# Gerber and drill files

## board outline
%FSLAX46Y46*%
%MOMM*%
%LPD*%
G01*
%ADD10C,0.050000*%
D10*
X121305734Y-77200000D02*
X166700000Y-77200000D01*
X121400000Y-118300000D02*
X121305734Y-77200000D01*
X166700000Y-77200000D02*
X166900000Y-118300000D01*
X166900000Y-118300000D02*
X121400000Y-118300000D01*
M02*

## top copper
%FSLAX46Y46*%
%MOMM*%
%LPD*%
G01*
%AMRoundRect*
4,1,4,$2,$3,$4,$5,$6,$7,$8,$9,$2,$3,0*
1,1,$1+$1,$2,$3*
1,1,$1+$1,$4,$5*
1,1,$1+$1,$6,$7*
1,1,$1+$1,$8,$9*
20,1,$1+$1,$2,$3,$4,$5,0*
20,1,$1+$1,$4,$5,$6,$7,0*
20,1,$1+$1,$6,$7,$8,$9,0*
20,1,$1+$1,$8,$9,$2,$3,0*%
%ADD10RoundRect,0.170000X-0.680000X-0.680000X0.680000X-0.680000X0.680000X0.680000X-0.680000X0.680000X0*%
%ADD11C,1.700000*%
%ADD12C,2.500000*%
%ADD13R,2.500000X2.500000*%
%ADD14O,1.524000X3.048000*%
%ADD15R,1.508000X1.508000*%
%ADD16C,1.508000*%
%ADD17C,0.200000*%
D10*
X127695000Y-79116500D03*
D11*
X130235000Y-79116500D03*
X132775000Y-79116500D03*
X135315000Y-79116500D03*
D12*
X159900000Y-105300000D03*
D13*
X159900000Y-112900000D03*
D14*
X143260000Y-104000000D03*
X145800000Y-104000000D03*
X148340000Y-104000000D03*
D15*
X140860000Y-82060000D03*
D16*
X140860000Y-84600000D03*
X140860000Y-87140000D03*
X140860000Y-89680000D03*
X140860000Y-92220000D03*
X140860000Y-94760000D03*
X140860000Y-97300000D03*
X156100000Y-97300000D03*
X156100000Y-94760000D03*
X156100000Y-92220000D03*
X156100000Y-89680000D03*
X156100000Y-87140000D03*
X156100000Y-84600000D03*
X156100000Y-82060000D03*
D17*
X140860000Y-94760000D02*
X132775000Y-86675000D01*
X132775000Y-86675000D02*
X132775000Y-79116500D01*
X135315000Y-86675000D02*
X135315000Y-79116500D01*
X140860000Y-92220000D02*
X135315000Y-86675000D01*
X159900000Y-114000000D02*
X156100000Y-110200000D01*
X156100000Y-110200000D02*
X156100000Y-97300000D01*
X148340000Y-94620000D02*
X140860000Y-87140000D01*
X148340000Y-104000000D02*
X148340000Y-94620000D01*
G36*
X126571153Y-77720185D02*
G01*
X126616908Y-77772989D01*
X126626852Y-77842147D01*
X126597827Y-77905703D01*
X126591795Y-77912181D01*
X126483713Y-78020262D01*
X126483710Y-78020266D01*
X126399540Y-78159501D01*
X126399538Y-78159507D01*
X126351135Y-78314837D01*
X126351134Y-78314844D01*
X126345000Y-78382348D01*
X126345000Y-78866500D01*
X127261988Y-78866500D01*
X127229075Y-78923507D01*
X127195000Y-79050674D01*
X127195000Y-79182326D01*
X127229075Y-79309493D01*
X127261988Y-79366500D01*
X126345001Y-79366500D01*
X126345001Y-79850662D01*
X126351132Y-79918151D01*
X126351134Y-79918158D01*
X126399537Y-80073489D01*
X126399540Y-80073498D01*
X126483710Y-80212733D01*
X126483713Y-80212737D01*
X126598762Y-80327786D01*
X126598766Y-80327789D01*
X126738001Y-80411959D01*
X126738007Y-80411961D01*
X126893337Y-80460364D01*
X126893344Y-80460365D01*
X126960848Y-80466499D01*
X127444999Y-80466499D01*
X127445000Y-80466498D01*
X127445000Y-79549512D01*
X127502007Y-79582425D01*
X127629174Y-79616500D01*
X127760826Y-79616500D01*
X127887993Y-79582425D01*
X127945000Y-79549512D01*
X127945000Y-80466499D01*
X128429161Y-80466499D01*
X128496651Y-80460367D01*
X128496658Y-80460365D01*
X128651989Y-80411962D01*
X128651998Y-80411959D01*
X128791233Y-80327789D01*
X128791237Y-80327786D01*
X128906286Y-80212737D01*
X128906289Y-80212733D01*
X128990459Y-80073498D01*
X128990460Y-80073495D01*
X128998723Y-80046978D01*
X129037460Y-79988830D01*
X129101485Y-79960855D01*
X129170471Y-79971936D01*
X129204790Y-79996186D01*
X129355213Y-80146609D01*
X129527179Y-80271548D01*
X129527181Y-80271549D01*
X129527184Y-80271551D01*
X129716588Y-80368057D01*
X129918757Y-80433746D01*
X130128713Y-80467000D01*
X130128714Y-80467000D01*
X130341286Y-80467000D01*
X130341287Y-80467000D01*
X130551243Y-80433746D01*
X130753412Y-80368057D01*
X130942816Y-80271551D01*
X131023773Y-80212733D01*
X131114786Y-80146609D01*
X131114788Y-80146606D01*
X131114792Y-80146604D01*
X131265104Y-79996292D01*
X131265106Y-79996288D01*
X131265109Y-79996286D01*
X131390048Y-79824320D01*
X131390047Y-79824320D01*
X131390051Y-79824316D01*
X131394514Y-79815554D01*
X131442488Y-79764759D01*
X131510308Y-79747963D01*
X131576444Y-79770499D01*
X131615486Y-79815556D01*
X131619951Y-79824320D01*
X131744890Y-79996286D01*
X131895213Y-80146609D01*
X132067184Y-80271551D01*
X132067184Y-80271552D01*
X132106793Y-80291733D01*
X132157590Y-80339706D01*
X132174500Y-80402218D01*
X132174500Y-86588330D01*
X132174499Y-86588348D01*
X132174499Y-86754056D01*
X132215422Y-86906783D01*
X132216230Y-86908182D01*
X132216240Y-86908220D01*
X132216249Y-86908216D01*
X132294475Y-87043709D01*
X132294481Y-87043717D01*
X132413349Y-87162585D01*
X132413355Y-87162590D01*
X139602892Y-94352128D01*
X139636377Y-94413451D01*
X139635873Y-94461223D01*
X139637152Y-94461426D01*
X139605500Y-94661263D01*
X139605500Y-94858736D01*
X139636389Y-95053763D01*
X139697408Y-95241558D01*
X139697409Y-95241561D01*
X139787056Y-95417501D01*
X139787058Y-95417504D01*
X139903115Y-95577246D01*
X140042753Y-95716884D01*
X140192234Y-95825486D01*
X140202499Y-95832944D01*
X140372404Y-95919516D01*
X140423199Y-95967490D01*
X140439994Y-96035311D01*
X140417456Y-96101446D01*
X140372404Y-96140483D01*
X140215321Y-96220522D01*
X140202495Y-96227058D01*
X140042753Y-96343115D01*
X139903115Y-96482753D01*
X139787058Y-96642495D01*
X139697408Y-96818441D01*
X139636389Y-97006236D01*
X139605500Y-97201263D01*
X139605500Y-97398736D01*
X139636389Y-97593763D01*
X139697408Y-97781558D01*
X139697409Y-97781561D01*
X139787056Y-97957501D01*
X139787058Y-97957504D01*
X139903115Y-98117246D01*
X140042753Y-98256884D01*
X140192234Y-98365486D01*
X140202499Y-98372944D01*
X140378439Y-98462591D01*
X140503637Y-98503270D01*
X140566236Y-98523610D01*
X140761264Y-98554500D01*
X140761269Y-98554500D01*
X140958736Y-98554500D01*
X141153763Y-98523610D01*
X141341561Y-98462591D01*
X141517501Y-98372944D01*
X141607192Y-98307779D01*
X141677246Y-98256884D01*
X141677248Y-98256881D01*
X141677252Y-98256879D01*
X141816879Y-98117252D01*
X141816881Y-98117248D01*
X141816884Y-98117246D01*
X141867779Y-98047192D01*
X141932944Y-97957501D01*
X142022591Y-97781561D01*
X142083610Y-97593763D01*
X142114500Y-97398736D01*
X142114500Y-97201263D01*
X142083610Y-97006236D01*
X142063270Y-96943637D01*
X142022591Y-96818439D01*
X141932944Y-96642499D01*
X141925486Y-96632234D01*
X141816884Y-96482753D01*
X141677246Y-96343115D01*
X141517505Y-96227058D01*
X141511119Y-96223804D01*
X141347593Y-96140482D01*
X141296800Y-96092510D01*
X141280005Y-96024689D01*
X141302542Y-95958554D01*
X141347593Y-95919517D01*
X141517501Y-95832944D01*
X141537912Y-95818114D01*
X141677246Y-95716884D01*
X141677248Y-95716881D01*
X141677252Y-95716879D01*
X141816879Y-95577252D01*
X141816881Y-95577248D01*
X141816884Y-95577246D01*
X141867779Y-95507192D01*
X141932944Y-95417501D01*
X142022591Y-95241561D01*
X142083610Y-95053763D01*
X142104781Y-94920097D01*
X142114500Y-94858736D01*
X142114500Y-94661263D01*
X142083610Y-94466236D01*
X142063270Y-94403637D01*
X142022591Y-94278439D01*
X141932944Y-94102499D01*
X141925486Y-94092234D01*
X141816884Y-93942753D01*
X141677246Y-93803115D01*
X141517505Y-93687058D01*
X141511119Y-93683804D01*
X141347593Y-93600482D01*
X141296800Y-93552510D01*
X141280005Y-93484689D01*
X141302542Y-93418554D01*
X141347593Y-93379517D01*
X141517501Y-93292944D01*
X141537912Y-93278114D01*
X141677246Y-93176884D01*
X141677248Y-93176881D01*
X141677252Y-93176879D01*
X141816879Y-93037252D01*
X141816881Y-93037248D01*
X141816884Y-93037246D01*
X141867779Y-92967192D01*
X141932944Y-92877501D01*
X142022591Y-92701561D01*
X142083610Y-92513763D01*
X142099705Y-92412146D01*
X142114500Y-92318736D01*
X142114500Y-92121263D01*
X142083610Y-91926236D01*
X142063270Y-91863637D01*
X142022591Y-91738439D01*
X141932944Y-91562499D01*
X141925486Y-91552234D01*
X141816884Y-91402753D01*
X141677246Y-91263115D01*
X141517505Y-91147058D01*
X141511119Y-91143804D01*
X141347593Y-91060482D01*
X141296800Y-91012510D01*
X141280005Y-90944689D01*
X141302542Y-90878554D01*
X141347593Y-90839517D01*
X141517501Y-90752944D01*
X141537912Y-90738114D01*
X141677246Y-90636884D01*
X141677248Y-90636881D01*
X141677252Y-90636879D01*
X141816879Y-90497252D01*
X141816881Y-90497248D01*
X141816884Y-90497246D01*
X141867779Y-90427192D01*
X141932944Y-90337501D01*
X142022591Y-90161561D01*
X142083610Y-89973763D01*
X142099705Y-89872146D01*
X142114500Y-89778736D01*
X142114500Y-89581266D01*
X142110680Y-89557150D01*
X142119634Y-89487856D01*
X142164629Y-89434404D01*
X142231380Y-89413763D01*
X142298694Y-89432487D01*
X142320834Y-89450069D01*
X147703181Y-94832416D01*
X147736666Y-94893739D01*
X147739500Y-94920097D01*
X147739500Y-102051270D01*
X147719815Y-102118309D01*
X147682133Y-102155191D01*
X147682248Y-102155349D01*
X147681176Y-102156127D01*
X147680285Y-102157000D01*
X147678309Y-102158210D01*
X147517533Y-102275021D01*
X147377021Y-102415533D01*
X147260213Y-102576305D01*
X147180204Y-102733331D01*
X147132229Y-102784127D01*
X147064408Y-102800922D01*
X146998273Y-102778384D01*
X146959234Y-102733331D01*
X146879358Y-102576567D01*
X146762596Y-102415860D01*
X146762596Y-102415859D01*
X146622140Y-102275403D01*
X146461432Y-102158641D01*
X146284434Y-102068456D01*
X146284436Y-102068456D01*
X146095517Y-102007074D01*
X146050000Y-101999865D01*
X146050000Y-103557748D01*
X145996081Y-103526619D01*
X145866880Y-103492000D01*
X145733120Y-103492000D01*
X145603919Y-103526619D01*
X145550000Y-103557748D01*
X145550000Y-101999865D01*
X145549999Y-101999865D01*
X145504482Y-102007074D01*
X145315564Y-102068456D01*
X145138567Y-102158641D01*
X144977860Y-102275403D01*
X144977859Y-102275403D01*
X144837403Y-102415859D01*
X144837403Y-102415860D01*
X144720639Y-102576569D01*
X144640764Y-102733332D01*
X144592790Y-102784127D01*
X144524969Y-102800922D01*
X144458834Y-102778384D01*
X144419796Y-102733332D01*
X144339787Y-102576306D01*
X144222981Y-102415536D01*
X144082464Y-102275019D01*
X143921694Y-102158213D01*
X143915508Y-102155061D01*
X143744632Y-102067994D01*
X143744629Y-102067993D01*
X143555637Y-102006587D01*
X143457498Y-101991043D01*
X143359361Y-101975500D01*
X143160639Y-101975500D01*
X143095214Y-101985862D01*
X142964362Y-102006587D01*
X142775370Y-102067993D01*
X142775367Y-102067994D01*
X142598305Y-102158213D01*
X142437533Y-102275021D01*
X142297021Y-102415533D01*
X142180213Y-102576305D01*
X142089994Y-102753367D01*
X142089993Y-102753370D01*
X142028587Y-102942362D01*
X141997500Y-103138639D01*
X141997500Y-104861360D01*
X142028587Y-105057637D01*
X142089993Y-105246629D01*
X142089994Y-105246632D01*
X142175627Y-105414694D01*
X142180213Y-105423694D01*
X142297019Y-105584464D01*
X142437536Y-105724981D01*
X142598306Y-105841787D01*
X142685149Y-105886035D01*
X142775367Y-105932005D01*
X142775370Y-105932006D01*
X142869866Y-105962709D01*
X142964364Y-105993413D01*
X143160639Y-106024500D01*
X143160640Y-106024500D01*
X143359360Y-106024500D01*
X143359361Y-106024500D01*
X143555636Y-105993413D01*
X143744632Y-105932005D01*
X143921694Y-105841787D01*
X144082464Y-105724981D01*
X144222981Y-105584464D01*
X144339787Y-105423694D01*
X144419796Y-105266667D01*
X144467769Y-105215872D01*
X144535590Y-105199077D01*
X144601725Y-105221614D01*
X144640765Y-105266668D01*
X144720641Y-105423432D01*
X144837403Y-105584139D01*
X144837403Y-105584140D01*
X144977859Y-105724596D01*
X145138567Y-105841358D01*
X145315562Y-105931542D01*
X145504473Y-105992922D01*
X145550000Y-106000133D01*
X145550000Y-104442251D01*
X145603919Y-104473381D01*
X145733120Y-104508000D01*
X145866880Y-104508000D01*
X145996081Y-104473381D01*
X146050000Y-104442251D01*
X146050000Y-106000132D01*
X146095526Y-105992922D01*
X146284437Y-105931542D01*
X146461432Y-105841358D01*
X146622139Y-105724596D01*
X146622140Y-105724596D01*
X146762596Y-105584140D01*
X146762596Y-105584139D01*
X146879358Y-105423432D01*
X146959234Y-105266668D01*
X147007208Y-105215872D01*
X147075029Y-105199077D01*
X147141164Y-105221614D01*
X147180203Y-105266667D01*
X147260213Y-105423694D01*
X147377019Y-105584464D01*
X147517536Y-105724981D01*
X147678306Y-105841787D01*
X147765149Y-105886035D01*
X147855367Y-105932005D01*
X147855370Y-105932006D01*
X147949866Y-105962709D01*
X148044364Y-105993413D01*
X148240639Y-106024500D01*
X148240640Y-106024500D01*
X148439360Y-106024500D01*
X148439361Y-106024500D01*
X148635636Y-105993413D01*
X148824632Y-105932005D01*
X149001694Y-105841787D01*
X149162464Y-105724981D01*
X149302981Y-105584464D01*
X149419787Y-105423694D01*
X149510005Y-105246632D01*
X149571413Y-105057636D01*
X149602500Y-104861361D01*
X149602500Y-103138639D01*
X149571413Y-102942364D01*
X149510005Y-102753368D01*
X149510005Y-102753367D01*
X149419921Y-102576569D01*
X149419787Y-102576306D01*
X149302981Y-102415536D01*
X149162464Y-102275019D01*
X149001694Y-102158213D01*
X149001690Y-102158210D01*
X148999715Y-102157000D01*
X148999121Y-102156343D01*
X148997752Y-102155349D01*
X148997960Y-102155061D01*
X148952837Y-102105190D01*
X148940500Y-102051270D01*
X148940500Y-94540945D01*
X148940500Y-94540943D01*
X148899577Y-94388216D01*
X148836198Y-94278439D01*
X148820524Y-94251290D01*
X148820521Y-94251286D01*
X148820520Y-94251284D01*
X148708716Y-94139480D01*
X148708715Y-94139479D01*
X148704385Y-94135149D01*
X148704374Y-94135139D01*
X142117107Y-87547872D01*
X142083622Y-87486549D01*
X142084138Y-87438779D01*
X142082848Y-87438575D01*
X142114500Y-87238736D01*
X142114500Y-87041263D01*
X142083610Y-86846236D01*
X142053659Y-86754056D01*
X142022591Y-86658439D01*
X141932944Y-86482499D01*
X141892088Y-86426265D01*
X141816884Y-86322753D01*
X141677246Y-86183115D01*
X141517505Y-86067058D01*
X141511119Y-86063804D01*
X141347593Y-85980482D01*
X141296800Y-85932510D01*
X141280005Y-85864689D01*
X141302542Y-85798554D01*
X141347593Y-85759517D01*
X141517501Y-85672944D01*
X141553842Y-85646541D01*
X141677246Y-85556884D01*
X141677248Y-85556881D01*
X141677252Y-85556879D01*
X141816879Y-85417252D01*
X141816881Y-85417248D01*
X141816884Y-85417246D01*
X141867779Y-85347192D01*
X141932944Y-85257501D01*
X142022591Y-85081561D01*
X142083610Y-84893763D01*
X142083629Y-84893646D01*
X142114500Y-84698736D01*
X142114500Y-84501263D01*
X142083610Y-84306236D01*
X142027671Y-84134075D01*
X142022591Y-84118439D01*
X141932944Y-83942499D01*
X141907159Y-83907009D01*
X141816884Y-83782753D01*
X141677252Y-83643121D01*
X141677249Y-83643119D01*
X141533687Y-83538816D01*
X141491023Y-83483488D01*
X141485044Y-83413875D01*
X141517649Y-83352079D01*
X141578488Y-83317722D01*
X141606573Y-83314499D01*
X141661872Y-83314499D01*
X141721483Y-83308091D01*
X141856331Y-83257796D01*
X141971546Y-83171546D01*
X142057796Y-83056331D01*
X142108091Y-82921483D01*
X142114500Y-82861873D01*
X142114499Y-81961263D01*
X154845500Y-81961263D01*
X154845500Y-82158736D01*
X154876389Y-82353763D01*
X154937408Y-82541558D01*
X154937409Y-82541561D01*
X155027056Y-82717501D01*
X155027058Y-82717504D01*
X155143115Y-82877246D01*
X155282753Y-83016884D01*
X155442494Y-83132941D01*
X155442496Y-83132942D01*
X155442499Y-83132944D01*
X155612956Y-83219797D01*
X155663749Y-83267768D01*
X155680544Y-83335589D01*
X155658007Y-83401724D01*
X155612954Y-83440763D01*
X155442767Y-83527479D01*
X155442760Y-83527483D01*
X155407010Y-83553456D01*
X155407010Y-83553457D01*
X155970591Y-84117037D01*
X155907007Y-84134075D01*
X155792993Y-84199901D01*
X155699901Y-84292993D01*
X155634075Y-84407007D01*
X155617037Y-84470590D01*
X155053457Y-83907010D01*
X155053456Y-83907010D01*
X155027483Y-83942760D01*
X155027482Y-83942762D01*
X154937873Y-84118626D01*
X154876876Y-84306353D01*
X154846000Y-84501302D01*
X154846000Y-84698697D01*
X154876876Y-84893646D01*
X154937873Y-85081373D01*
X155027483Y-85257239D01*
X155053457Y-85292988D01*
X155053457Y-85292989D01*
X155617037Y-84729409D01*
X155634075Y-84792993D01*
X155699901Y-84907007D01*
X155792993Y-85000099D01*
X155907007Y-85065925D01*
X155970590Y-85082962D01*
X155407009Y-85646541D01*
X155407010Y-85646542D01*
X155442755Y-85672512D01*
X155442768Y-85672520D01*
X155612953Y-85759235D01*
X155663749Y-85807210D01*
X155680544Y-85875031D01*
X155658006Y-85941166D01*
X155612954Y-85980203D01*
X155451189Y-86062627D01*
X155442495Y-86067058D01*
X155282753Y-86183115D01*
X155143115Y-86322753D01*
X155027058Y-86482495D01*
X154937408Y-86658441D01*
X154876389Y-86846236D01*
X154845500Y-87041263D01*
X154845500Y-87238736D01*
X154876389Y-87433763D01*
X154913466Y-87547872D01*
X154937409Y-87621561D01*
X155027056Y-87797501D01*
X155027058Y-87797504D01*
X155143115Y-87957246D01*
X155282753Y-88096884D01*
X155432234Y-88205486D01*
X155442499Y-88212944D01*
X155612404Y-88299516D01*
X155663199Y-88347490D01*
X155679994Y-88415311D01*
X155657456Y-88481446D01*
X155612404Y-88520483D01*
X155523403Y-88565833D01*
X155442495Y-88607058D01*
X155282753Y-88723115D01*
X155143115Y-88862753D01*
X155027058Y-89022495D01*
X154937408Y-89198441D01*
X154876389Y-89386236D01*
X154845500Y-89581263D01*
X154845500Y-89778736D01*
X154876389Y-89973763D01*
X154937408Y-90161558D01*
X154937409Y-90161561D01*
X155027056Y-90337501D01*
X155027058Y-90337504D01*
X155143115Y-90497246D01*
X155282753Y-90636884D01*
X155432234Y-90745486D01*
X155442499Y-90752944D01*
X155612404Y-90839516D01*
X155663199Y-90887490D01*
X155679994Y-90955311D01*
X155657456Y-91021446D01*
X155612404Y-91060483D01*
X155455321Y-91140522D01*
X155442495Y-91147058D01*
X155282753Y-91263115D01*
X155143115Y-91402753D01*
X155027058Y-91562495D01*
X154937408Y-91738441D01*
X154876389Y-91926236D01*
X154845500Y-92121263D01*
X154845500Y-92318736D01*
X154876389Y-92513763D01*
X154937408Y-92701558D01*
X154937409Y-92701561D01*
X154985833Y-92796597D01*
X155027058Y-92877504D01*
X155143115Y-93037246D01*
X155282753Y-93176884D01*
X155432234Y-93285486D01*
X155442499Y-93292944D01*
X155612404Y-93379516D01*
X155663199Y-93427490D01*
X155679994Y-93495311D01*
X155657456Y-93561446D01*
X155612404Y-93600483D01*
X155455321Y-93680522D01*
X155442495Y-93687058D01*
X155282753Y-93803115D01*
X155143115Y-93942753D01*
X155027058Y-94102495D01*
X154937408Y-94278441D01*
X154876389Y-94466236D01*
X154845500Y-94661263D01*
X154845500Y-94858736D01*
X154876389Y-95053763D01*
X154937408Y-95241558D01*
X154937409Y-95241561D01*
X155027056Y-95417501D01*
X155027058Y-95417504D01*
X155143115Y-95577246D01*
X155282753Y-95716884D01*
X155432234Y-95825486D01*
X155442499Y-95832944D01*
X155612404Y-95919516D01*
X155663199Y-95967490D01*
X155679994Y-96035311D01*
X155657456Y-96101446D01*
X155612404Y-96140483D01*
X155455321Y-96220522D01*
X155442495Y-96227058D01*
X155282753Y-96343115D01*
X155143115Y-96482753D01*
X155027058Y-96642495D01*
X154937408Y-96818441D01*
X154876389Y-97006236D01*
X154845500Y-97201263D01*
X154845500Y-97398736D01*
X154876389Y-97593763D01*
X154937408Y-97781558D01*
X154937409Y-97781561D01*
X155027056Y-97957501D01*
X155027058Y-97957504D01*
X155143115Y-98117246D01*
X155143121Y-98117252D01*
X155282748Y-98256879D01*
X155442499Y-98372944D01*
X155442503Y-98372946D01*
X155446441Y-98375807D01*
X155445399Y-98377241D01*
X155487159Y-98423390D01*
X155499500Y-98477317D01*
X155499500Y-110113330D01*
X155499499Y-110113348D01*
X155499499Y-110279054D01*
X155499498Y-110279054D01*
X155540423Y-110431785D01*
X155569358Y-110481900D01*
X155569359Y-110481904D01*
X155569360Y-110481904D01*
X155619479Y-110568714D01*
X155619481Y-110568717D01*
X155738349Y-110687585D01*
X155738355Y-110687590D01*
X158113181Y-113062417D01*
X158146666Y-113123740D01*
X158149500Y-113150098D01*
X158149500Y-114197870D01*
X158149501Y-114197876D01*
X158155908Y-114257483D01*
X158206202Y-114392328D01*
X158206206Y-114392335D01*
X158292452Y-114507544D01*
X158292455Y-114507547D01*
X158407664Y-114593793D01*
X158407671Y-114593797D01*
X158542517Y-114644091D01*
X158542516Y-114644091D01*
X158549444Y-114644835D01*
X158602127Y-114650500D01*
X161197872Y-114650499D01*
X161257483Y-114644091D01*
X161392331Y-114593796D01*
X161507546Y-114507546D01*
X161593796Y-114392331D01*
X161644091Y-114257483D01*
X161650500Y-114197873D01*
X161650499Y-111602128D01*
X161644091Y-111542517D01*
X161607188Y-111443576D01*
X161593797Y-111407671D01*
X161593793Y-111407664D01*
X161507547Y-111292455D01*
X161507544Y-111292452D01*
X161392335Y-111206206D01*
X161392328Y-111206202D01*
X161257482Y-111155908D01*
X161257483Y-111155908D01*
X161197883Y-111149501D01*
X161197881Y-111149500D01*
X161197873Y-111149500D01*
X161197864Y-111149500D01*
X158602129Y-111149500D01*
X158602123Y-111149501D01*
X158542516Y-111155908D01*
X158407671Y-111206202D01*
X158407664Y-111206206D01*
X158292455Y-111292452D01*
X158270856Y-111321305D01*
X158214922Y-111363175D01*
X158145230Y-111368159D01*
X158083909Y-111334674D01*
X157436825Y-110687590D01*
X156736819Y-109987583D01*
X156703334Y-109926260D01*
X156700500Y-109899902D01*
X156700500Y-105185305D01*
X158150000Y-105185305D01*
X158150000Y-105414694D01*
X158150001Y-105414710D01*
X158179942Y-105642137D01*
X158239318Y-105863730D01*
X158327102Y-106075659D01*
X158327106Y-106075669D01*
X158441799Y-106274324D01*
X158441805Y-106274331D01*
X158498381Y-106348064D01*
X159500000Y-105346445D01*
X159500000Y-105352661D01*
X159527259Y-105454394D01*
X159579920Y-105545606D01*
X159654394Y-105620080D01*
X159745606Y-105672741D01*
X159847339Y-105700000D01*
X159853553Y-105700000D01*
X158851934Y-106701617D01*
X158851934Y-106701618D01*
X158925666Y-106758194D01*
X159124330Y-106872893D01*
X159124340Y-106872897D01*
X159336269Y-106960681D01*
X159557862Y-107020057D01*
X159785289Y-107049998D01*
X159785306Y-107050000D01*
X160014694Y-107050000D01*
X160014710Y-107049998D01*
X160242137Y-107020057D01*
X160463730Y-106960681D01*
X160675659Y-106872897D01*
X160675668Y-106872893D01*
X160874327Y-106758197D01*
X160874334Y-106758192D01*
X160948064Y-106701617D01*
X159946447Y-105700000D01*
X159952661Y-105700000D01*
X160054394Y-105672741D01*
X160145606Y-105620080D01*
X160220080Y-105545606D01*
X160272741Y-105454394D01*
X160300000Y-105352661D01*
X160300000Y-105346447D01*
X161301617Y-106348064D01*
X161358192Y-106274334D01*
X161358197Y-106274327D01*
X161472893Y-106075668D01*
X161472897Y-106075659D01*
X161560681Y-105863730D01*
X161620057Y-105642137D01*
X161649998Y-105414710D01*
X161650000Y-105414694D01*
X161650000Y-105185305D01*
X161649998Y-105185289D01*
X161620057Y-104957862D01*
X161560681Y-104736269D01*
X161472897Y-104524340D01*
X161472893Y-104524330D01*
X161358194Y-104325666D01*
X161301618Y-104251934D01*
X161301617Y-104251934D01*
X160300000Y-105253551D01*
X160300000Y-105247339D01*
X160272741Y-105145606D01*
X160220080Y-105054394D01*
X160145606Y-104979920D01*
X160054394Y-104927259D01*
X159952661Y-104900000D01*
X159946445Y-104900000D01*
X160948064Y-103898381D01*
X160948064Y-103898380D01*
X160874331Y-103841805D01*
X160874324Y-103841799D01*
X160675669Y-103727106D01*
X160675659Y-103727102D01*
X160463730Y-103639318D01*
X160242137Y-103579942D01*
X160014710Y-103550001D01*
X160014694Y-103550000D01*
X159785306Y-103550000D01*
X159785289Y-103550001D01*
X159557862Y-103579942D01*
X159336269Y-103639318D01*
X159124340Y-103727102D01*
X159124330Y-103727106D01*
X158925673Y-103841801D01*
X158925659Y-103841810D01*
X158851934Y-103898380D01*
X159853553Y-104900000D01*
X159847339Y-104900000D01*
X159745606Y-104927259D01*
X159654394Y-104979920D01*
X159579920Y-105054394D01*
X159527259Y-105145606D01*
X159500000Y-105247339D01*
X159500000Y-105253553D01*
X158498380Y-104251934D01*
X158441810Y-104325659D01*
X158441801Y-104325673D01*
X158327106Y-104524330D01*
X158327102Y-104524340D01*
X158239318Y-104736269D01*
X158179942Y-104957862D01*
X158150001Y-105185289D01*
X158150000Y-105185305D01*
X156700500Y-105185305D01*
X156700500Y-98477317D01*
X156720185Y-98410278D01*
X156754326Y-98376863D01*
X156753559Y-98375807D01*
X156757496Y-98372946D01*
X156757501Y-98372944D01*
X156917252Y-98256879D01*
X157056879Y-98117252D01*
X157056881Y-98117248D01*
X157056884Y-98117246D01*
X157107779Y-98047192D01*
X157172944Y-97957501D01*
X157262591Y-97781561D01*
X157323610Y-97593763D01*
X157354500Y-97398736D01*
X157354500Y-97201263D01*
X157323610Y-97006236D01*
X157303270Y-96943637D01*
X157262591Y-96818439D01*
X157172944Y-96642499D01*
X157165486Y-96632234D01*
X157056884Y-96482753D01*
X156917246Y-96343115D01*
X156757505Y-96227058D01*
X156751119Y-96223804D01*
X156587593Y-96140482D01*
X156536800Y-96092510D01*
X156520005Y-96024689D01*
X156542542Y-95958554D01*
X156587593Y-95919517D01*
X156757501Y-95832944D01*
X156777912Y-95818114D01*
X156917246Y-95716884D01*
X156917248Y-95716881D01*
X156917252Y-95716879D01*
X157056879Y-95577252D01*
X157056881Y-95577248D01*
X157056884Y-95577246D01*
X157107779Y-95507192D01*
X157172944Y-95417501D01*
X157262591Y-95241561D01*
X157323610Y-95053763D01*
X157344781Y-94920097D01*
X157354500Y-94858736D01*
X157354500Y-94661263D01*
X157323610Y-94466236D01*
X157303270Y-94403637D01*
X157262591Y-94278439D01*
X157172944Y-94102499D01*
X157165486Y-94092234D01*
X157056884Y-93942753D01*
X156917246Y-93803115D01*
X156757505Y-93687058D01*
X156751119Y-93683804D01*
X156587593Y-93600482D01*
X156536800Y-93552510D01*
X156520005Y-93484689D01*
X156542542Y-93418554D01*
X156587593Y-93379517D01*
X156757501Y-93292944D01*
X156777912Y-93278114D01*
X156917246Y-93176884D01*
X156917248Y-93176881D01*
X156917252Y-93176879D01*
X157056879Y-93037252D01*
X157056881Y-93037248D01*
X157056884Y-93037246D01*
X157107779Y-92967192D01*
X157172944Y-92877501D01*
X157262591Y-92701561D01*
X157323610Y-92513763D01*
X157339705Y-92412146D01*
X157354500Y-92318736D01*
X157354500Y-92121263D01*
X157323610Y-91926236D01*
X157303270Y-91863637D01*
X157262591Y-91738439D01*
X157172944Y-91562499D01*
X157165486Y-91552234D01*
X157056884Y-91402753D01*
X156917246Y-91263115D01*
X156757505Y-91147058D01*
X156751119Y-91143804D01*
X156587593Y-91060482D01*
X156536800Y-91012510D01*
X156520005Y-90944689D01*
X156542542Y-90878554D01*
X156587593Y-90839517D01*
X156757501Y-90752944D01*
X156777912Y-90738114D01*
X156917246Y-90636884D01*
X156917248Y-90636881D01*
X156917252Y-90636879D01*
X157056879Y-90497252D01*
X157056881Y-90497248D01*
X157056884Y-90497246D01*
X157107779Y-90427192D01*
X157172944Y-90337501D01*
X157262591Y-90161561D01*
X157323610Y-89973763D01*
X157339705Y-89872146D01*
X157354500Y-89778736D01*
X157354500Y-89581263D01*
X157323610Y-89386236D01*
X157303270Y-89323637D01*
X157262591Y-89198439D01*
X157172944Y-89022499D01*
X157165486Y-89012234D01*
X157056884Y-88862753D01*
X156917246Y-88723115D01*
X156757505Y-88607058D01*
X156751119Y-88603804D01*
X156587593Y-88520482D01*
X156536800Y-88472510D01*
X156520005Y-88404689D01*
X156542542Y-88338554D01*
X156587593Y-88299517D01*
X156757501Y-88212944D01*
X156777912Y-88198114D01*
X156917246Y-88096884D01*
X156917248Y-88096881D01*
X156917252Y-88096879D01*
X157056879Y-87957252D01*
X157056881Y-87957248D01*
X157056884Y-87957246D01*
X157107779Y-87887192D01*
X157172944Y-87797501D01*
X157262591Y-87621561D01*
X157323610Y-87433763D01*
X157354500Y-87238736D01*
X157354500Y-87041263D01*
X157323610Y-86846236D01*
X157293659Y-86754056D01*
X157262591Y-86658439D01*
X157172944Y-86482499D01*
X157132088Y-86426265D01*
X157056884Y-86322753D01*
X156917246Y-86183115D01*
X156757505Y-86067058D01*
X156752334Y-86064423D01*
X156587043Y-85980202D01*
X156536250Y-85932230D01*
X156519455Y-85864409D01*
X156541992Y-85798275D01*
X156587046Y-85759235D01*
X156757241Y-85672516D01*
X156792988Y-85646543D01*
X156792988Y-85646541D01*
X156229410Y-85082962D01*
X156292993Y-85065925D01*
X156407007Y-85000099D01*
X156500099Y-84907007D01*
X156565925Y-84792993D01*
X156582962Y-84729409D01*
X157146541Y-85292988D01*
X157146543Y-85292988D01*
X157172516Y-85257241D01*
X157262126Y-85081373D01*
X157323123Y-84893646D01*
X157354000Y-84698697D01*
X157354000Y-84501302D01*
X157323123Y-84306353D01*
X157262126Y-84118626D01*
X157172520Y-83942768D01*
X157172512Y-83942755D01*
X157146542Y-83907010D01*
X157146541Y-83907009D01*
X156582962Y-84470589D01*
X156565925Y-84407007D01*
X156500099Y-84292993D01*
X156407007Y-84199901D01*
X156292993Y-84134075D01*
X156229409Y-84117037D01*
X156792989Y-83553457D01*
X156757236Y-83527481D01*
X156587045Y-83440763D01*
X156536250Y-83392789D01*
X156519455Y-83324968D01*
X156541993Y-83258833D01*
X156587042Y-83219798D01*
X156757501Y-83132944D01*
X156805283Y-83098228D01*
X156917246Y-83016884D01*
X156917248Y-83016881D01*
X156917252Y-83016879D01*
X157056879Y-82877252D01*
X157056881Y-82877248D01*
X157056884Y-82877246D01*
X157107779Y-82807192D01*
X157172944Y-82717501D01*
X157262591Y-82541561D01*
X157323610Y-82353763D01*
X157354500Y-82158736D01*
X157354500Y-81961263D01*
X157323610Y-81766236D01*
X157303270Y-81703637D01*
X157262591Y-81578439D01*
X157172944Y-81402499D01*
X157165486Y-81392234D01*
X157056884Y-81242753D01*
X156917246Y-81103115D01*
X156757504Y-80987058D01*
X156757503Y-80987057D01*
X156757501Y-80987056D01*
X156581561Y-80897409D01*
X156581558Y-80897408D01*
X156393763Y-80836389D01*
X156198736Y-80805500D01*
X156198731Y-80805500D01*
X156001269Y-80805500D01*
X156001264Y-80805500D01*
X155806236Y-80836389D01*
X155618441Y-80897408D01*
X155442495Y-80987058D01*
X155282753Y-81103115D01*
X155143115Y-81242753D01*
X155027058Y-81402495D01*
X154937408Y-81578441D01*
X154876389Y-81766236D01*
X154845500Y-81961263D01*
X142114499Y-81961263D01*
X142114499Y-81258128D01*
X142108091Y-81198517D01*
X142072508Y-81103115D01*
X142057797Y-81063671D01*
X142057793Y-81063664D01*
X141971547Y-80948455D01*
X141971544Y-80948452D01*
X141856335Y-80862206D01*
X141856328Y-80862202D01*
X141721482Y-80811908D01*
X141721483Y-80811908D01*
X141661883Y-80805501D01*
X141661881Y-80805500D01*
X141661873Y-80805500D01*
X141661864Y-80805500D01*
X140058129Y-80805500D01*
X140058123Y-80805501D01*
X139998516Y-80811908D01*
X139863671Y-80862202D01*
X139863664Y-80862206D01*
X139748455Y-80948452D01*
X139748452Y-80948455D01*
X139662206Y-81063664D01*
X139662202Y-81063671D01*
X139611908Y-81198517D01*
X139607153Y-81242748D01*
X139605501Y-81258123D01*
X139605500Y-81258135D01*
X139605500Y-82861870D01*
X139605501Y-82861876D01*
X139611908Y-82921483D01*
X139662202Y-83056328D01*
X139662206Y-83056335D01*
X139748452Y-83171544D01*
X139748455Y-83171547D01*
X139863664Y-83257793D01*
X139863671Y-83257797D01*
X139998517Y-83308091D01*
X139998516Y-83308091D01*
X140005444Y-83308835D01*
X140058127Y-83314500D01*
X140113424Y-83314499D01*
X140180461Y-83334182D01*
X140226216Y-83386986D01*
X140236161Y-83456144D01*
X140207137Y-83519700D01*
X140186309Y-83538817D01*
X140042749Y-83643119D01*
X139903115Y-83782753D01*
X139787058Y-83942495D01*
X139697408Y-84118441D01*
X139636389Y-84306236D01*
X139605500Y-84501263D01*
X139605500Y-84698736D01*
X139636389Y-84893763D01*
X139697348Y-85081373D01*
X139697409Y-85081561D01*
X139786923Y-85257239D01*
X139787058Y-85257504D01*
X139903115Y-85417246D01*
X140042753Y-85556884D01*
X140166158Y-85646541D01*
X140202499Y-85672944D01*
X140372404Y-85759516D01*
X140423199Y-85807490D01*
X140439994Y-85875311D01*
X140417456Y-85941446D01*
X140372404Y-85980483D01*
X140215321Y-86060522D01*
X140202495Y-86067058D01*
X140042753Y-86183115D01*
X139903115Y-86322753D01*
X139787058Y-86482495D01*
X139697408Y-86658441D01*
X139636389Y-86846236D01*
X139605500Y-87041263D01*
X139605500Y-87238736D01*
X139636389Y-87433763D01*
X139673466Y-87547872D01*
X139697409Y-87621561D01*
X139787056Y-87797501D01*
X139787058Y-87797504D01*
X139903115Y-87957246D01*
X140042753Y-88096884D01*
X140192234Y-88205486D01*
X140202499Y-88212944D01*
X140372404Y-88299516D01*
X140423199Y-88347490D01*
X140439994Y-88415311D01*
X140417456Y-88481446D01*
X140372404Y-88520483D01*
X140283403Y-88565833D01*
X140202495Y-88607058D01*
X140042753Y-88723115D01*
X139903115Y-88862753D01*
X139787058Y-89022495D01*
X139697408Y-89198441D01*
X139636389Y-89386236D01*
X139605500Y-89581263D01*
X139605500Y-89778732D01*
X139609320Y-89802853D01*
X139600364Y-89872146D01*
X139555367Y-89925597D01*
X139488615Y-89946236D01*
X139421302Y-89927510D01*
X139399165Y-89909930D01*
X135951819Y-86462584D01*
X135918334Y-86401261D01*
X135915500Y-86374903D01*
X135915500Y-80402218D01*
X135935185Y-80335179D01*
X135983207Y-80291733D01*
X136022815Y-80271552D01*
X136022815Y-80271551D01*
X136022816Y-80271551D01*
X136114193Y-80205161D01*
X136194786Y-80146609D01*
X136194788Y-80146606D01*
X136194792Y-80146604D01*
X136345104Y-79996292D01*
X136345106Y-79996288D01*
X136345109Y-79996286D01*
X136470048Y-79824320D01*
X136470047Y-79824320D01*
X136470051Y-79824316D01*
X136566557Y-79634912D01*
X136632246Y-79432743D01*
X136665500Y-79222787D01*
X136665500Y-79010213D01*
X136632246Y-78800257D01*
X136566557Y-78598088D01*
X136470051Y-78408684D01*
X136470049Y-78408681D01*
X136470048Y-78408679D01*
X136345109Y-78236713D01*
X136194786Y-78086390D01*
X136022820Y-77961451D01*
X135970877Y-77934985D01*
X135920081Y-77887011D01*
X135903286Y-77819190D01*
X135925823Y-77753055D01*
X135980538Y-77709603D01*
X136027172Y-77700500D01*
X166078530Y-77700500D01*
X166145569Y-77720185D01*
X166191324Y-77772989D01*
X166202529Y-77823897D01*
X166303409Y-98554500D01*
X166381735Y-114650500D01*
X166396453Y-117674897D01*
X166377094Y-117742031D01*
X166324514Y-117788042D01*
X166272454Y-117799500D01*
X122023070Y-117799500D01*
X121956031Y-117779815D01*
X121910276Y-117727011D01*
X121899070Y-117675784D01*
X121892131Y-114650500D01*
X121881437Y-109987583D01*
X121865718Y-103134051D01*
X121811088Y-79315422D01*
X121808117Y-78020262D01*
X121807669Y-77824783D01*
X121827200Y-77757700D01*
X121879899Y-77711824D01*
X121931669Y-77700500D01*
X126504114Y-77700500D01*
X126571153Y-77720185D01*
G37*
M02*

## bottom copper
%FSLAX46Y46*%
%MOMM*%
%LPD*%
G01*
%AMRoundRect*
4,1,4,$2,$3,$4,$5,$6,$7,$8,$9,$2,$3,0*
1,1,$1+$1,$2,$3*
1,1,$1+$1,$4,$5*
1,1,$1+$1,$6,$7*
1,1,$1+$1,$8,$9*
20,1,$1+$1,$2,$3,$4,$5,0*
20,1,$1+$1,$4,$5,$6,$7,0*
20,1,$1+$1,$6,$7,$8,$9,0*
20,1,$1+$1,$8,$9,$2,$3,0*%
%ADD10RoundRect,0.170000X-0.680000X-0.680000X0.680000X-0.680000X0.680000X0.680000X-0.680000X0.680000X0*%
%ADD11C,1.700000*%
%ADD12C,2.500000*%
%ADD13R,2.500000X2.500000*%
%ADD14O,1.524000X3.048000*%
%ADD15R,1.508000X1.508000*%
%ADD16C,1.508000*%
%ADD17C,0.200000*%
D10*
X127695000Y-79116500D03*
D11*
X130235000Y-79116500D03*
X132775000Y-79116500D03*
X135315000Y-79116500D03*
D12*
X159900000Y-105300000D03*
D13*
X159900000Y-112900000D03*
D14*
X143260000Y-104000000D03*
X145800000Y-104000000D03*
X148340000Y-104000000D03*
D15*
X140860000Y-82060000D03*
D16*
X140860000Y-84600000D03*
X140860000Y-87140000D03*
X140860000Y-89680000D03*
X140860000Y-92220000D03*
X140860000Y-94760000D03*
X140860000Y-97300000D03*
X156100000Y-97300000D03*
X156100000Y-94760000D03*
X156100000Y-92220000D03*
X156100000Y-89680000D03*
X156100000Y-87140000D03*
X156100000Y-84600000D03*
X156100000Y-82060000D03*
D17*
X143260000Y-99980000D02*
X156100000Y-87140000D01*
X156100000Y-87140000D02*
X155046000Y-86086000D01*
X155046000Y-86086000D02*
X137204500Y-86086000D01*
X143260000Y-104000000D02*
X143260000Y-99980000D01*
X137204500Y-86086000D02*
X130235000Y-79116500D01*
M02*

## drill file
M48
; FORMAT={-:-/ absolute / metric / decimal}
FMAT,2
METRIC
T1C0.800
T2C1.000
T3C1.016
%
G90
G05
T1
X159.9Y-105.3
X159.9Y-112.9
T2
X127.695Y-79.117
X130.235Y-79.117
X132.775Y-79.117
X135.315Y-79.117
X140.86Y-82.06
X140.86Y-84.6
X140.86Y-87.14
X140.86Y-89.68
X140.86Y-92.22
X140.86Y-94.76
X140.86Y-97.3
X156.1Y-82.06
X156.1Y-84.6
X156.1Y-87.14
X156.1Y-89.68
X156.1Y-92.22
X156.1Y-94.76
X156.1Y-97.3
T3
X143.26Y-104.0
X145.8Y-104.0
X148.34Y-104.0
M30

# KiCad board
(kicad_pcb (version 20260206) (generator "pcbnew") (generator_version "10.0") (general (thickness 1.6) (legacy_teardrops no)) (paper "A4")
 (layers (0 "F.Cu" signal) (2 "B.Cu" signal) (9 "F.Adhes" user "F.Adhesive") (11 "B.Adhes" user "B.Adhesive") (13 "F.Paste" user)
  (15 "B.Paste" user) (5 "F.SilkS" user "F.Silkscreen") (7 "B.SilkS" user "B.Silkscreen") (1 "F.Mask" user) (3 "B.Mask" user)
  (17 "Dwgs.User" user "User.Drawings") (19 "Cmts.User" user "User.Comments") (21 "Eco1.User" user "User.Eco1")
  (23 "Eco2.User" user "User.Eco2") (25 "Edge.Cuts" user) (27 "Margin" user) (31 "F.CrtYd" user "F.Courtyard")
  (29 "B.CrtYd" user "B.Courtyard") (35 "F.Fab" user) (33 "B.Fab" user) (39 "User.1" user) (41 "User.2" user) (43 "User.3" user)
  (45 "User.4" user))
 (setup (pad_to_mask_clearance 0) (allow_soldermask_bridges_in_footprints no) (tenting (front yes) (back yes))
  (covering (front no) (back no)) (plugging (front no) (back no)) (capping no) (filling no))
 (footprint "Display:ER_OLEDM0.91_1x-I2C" (layer "F.Cu") (at 127.695 79.1165)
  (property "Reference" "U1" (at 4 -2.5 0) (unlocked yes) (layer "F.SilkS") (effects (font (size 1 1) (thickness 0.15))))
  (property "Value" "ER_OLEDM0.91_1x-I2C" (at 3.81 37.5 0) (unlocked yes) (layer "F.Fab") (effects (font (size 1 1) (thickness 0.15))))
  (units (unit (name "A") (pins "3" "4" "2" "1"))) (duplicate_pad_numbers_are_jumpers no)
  (pad "1" thru_hole roundrect (at 0 0) (size 1.7 1.7) (drill 1) (layers "*.Cu" "*.Mask") (remove_unused_layers no) (roundrect_rratio 0.1)
   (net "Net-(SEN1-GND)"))
  (pad "2" thru_hole circle (at 2.54 0) (size 1.7 1.7) (drill 1) (layers "*.Cu" "*.Mask") (remove_unused_layers no) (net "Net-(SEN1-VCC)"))
  (pad "3" thru_hole circle (at 5.08 0) (size 1.7 1.7) (drill 1) (layers "*.Cu" "*.Mask") (remove_unused_layers no) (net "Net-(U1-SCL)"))
  (pad "4" thru_hole circle (at 7.62 0) (size 1.7 1.7) (drill 1) (layers "*.Cu" "*.Mask") (remove_unused_layers no) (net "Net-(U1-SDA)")))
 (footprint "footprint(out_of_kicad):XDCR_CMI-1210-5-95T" (layer "F.Cu") (at 159.9 109.1 90)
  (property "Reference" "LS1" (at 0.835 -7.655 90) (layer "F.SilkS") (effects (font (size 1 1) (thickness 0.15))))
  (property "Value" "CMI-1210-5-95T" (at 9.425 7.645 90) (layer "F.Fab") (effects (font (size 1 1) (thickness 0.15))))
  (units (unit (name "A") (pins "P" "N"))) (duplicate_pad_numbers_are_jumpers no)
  (pad "N" thru_hole circle (at 3.8 0 90) (size 2.5 2.5) (drill 0.8) (layers "*.Cu" "*.Mask") (remove_unused_layers no)
   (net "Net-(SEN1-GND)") (solder_mask_margin 0.102))
  (pad "P" thru_hole rect (at -3.8 0 90) (size 2.5 2.5) (drill 0.8) (layers "*.Cu" "*.Mask") (remove_unused_layers no)
   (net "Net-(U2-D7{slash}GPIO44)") (solder_mask_margin 0.102)))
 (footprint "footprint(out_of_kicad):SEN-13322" (layer "F.Cu") (at 145.8 104)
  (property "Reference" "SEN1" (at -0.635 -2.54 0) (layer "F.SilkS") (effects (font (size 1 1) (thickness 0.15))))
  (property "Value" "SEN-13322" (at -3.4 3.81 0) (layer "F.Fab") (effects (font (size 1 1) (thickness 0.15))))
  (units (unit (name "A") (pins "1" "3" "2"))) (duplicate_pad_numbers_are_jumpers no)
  (pad "1" thru_hole oval (at -2.54 0) (size 1.524 3.048) (drill 1.016) (layers "*.Cu" "*.Mask") (remove_unused_layers no)
   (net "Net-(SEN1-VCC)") (solder_mask_margin 0.102))
  (pad "2" thru_hole oval (at 0 0) (size 1.524 3.048) (drill 1.016) (layers "*.Cu" "*.Mask") (remove_unused_layers no)
   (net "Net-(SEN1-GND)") (solder_mask_margin 0.102))
  (pad "3" thru_hole oval (at 2.54 0) (size 1.524 3.048) (drill 1.016) (layers "*.Cu" "*.Mask") (remove_unused_layers no)
   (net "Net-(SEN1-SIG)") (solder_mask_margin 0.102)))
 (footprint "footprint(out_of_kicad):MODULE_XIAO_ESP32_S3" (layer "F.Cu") (at 148.48 89.6165)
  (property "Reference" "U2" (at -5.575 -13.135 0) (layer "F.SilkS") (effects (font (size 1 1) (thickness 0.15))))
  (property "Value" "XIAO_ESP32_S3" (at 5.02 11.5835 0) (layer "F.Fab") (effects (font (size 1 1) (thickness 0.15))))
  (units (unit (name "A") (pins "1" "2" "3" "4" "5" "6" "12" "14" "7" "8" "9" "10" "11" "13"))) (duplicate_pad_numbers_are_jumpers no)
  (pad "1" thru_hole rect (at -7.62 -7.5565) (size 1.508 1.508) (drill 1) (layers "*.Cu" "*.Mask") (remove_unused_layers no)
   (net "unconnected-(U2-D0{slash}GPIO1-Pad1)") (solder_mask_margin 0.102))
  (pad "2" thru_hole circle (at -7.62 -5.0165) (size 1.508 1.508) (drill 1) (layers "*.Cu" "*.Mask") (remove_unused_layers no)
   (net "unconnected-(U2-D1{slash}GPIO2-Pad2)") (solder_mask_margin 0.102))
  (pad "3" thru_hole circle (at -7.62 -2.4765) (size 1.508 1.508) (drill 1) (layers "*.Cu" "*.Mask") (remove_unused_layers no)
   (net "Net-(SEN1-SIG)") (solder_mask_margin 0.102))
  (pad "4" thru_hole circle (at -7.62 0.0635) (size 1.508 1.508) (drill 1) (layers "*.Cu" "*.Mask") (remove_unused_layers no)
   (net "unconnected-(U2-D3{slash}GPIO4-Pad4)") (solder_mask_margin 0.102))
  (pad "5" thru_hole circle (at -7.62 2.6035) (size 1.508 1.508) (drill 1) (layers "*.Cu" "*.Mask") (remove_unused_layers no)
   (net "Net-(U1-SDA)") (solder_mask_margin 0.102))
  (pad "6" thru_hole circle (at -7.62 5.1435) (size 1.508 1.508) (drill 1) (layers "*.Cu" "*.Mask") (remove_unused_layers no)
   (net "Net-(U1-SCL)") (solder_mask_margin 0.102))
  (pad "7" thru_hole circle (at -7.62 7.6835) (size 1.508 1.508) (drill 1) (layers "*.Cu" "*.Mask") (remove_unused_layers no)
   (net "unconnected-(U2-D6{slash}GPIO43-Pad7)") (solder_mask_margin 0.102))
  (pad "8" thru_hole circle (at 7.62 7.6835) (size 1.508 1.508) (drill 1) (layers "*.Cu" "*.Mask") (remove_unused_layers no)
   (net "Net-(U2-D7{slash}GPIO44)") (solder_mask_margin 0.102))
  (pad "9" thru_hole circle (at 7.62 5.1435) (size 1.508 1.508) (drill 1) (layers "*.Cu" "*.Mask") (remove_unused_layers no)
   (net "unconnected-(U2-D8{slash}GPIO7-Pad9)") (solder_mask_margin 0.102))
  (pad "10" thru_hole circle (at 7.62 2.6035) (size 1.508 1.508) (drill 1) (layers "*.Cu" "*.Mask") (remove_unused_layers no)
   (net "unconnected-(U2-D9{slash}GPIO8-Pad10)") (solder_mask_margin 0.102))
  (pad "11" thru_hole circle (at 7.62 0.0635) (size 1.508 1.508) (drill 1) (layers "*.Cu" "*.Mask") (remove_unused_layers no)
   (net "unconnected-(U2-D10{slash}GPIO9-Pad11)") (solder_mask_margin 0.102))
  (pad "12" thru_hole circle (at 7.62 -2.4765) (size 1.508 1.508) (drill 1) (layers "*.Cu" "*.Mask") (remove_unused_layers no)
   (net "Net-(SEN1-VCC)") (solder_mask_margin 0.102))
  (pad "13" thru_hole circle (at 7.62 -5.0165) (size 1.508 1.508) (drill 1) (layers "*.Cu" "*.Mask") (remove_unused_layers no)
   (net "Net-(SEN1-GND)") (solder_mask_margin 0.102))
  (pad "14" thru_hole circle (at 7.62 -7.5565) (size 1.508 1.508) (drill 1) (layers "*.Cu" "*.Mask") (remove_unused_layers no)
   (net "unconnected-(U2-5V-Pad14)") (solder_mask_margin 0.102)))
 (gr_line (start 121.305734 77.2) (end 166.7 77.2) (stroke (width 0.05) (type default)) (layer "Edge.Cuts"))
 (gr_line (start 121.4 118.3) (end 121.305734 77.2) (stroke (width 0.05) (type default)) (layer "Edge.Cuts"))
 (gr_line (start 166.7 77.2) (end 166.9 118.3) (stroke (width 0.05) (type default)) (layer "Edge.Cuts"))
 (gr_line (start 166.9 118.3) (end 121.4 118.3) (stroke (width 0.05) (type default)) (layer "Edge.Cuts"))
 (segment (start 143.26 99.98) (end 156.1 87.14) (width 0.2) (layer "B.Cu") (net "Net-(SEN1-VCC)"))
 (segment (start 156.1 87.14) (end 155.046 86.086) (width 0.2) (layer "B.Cu") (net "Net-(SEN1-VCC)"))
 (segment (start 155.046 86.086) (end 137.2045 86.086) (width 0.2) (layer "B.Cu") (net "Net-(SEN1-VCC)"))
 (segment (start 143.26 104) (end 143.26 99.98) (width 0.2) (layer "B.Cu") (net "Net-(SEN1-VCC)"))
 (segment (start 137.2045 86.086) (end 130.235 79.1165) (width 0.2) (layer "B.Cu") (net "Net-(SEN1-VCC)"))
 (segment (start 140.86 94.76) (end 132.775 86.675) (width 0.2) (layer "F.Cu") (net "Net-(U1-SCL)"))
 (segment (start 132.775 86.675) (end 132.775 79.1165) (width 0.2) (layer "F.Cu") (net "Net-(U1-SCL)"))
 (segment (start 135.315 86.675) (end 135.315 79.1165) (width 0.2) (layer "F.Cu") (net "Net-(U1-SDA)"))
 (segment (start 140.86 92.22) (end 135.315 86.675) (width 0.2) (layer "F.Cu") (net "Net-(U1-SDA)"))
 (segment (start 159.9 114) (end 156.1 110.2) (width 0.2) (layer "F.Cu") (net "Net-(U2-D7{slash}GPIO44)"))
 (segment (start 156.1 110.2) (end 156.1 97.3) (width 0.2) (layer "F.Cu") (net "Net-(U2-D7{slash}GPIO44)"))
 (segment (start 148.34 94.62) (end 140.86 87.14) (width 0.2) (layer "F.Cu") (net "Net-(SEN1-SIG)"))
 (segment (start 148.34 104) (end 148.34 94.62) (width 0.2) (layer "F.Cu") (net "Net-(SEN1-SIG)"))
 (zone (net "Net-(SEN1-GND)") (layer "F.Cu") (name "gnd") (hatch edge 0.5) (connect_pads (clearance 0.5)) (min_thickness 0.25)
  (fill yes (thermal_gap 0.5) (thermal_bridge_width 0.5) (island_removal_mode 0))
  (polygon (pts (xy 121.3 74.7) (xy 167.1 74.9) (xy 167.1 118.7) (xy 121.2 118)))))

